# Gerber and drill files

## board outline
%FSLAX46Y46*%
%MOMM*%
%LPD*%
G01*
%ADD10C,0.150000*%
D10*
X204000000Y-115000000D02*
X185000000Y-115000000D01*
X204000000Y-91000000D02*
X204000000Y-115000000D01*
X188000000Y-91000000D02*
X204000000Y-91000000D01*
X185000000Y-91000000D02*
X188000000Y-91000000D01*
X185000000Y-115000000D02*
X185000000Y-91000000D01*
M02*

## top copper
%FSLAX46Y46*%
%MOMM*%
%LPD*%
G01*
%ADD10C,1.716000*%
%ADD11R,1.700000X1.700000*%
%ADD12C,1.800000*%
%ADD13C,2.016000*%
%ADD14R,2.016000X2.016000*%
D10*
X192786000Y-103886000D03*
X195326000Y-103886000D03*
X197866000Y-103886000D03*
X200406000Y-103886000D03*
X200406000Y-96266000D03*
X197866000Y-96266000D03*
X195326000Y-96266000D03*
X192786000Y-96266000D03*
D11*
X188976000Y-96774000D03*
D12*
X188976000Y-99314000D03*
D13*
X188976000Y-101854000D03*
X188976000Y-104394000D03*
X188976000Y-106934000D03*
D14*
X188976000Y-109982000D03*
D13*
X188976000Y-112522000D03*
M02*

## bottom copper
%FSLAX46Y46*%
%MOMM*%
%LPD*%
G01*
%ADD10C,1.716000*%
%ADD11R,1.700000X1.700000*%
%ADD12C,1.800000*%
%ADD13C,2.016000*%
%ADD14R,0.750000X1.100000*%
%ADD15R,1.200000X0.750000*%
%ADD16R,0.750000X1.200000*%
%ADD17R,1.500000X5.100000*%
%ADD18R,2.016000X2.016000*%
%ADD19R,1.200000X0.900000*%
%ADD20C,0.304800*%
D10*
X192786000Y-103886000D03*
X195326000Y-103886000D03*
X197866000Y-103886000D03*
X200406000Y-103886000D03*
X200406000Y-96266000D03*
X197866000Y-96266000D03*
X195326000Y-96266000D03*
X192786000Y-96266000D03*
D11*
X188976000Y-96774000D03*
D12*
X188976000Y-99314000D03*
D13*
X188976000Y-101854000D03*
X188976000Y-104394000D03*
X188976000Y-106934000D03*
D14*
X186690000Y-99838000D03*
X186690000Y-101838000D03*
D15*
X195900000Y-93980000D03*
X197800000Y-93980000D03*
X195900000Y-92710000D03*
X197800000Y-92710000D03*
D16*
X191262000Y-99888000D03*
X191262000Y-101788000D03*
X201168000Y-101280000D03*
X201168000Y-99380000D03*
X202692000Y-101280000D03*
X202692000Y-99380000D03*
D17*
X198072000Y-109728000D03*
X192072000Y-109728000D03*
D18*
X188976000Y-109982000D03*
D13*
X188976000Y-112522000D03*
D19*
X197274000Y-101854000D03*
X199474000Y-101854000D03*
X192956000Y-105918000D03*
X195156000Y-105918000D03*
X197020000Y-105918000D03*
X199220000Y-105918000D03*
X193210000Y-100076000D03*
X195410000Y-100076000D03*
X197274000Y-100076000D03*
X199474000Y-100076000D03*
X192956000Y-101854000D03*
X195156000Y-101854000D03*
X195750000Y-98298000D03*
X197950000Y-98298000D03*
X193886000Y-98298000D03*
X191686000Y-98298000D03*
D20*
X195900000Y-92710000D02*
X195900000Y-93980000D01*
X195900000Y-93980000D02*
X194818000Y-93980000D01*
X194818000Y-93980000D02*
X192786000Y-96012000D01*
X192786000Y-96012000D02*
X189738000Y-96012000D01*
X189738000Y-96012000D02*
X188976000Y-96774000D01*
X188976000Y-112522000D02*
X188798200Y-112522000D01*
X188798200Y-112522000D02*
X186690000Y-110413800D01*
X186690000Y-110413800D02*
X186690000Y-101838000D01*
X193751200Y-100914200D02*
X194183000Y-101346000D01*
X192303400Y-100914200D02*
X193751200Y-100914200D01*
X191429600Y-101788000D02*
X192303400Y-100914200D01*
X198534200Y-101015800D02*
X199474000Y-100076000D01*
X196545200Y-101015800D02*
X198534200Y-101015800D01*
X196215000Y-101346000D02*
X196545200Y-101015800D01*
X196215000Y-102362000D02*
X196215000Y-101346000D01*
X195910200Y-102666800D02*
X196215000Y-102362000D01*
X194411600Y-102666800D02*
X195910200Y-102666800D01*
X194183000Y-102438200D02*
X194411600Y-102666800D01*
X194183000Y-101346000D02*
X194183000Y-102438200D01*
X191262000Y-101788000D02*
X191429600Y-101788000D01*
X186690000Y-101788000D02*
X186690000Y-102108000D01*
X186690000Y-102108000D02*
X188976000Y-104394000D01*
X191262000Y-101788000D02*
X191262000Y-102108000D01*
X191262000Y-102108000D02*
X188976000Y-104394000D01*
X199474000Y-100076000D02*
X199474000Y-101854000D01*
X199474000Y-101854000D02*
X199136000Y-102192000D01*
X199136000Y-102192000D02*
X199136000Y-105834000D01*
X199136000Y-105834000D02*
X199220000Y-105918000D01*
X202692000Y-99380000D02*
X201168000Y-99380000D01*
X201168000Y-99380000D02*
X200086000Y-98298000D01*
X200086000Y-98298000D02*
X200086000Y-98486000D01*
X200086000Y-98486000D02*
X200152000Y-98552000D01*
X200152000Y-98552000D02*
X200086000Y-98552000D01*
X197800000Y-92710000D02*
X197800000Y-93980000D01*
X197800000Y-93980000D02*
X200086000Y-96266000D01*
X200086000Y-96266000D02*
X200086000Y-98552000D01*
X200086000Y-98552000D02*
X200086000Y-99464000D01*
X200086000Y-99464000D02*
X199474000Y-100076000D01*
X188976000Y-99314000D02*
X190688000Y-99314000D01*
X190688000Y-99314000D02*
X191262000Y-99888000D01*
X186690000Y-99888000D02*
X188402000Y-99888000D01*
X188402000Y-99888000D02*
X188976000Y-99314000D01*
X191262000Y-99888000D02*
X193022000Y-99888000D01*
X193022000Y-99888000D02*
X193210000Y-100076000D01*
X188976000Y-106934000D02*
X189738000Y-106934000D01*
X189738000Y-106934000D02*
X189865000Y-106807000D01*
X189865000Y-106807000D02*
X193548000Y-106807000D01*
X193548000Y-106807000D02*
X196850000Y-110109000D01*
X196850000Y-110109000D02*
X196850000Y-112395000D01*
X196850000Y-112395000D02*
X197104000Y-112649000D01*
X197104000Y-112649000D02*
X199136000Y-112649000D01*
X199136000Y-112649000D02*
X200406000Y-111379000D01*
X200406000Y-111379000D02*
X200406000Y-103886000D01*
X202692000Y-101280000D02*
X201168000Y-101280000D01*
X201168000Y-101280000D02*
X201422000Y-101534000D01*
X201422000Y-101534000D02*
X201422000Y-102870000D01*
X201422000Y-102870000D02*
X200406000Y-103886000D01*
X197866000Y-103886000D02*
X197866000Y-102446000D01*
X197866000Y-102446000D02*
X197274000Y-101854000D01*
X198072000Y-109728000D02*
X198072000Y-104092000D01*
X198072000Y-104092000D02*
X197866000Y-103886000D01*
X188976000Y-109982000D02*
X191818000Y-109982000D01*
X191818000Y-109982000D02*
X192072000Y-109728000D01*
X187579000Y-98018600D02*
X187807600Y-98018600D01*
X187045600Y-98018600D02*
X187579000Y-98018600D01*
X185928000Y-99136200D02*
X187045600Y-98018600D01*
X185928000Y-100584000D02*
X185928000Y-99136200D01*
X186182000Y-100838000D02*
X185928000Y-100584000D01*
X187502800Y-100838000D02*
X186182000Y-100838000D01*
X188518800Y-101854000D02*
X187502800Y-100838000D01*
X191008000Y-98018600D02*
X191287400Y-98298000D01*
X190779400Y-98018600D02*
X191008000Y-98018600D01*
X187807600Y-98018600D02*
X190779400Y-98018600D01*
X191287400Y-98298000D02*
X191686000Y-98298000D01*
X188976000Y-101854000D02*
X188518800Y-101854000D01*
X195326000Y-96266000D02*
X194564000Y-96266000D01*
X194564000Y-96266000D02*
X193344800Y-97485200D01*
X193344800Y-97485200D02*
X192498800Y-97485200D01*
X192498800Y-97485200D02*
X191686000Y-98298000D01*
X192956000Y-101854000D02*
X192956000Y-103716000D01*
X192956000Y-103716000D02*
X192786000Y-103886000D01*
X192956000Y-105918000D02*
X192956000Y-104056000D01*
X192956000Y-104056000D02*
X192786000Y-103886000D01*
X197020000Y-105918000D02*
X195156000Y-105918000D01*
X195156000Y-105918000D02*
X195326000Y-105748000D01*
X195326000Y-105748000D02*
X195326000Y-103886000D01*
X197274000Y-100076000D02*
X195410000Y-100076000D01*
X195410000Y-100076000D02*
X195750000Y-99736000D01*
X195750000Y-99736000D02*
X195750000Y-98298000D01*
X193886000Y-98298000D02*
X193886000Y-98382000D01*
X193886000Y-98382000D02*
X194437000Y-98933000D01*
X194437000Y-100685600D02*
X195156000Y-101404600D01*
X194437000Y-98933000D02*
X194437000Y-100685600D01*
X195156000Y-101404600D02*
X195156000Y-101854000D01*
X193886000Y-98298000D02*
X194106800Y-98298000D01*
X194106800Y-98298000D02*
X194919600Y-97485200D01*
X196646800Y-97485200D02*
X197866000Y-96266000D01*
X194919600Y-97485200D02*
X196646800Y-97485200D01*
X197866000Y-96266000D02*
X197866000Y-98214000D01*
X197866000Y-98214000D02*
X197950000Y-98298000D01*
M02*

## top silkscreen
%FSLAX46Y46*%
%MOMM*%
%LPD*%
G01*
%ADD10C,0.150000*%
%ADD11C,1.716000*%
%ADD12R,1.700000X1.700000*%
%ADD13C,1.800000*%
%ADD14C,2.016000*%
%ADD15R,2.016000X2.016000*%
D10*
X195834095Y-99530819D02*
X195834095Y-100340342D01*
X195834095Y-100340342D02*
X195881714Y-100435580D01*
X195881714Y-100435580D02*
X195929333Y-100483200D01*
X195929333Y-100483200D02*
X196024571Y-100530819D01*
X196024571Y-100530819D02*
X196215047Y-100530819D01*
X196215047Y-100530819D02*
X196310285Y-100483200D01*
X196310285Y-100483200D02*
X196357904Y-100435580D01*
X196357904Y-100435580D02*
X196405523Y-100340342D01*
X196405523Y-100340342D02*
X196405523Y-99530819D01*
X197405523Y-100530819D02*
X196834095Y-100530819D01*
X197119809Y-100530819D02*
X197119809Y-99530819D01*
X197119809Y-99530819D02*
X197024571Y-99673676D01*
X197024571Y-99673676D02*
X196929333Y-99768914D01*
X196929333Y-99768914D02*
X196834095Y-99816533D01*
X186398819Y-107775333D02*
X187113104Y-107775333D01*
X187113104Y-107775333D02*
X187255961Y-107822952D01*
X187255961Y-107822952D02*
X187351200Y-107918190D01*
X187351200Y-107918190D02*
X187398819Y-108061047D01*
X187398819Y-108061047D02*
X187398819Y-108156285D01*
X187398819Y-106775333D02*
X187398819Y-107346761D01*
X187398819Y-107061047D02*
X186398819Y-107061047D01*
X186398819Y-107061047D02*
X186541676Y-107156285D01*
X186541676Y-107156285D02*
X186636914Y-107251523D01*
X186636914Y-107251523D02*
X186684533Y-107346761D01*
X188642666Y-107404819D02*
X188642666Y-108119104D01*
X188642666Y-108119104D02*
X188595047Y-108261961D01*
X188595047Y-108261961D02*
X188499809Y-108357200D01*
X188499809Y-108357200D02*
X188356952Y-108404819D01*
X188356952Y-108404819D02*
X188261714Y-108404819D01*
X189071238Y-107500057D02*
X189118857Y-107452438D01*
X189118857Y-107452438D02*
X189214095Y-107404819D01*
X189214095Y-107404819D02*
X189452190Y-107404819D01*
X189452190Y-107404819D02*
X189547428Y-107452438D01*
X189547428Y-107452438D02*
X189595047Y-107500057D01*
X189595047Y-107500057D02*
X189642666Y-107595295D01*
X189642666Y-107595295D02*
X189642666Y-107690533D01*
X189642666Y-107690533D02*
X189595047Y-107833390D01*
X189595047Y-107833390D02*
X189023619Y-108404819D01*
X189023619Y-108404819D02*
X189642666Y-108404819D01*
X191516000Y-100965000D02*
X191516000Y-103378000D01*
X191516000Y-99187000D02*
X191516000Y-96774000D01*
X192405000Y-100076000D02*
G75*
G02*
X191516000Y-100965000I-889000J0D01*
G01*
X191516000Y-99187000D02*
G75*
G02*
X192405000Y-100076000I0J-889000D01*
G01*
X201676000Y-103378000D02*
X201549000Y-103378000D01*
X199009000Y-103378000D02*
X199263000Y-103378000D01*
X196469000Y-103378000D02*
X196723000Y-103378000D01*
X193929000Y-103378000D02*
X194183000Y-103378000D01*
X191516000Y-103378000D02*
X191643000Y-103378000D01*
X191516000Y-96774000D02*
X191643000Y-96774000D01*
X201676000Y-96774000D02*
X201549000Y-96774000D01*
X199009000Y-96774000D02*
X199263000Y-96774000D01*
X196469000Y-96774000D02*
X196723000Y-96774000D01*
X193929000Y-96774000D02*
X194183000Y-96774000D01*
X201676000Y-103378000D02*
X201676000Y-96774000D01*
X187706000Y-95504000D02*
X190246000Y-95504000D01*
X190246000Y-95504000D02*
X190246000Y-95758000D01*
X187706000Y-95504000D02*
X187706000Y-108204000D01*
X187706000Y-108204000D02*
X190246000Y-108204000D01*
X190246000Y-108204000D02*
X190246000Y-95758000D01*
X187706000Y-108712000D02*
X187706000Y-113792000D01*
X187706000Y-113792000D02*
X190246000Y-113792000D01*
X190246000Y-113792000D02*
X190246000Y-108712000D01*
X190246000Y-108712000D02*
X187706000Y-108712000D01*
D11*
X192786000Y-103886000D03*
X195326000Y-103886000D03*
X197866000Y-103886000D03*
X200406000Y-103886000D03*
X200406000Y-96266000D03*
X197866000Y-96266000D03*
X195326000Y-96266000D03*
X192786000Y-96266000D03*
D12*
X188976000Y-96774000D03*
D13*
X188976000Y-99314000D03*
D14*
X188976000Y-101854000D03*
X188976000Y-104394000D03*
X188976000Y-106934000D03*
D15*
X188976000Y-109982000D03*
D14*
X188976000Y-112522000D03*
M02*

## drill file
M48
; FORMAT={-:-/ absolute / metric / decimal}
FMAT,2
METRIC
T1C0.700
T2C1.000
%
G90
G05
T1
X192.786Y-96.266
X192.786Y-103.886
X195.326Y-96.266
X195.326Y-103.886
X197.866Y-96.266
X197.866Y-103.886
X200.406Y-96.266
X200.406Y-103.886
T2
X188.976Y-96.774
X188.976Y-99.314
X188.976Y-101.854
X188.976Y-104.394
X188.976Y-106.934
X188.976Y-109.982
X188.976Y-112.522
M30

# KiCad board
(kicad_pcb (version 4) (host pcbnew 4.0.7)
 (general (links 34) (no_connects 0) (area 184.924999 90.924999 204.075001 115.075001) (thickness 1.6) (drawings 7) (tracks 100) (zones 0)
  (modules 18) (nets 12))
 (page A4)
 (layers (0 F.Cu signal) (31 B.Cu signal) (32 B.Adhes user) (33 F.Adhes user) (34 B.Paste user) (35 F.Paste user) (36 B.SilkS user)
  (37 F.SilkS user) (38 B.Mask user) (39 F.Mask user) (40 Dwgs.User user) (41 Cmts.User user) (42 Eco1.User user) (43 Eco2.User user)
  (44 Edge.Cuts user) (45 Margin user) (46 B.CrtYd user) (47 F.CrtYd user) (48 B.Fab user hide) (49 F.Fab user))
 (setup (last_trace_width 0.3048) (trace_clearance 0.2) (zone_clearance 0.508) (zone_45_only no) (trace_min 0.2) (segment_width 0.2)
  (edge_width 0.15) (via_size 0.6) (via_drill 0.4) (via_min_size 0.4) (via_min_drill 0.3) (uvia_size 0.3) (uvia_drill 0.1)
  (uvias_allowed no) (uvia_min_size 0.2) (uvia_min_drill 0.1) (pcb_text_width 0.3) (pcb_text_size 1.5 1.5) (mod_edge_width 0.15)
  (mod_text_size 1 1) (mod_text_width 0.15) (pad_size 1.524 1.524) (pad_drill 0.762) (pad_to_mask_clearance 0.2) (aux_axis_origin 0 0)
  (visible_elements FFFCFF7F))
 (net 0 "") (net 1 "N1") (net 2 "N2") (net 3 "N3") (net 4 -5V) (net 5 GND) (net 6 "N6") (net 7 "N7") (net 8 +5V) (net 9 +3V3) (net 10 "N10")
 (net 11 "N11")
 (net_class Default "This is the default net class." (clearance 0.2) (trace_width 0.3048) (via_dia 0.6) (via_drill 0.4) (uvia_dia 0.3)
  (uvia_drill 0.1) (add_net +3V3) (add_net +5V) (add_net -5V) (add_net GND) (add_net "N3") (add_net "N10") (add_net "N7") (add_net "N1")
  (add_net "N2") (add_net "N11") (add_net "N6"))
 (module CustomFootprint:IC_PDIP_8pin (layer F.Cu) (at 196.596 100.076)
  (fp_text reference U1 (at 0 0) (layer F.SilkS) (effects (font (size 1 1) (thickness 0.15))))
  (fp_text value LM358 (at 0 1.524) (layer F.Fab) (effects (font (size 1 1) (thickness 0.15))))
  (fp_line (start -5.08 0.889) (end -5.08 3.302) (layer F.SilkS) (width 0.15))
  (fp_line (start -5.08 -0.889) (end -5.08 -3.302) (layer F.SilkS) (width 0.15))
  (fp_arc (start -5.08 0) (end -4.191 0) (angle 90) (layer F.SilkS) (width 0.15))
  (fp_arc (start -5.08 0) (end -5.08 -0.889) (angle 90) (layer F.SilkS) (width 0.15))
  (fp_line (start 5.08 3.302) (end 4.953 3.302) (layer F.SilkS) (width 0.15))
  (fp_line (start 2.413 3.302) (end 2.667 3.302) (layer F.SilkS) (width 0.15))
  (fp_line (start -0.127 3.302) (end 0.127 3.302) (layer F.SilkS) (width 0.15))
  (fp_line (start -2.667 3.302) (end -2.413 3.302) (layer F.SilkS) (width 0.15))
  (fp_line (start -5.08 3.302) (end -4.953 3.302) (layer F.SilkS) (width 0.15))
  (fp_line (start -5.08 -3.302) (end -4.953 -3.302) (layer F.SilkS) (width 0.15))
  (fp_line (start 5.08 -3.302) (end 4.953 -3.302) (layer F.SilkS) (width 0.15))
  (fp_line (start 2.413 -3.302) (end 2.667 -3.302) (layer F.SilkS) (width 0.15))
  (fp_line (start -0.127 -3.302) (end 0.127 -3.302) (layer F.SilkS) (width 0.15))
  (fp_line (start -2.667 -3.302) (end -2.413 -3.302) (layer F.SilkS) (width 0.15))
  (fp_line (start 5.08 3.302) (end 5.08 -3.302) (layer F.SilkS) (width 0.15))
  (pad 1 thru_hole circle (at -3.81 3.81) (size 1.716 1.716) (drill 0.7) (layers *.Cu *.Mask F.SilkS) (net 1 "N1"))
  (pad 2 thru_hole circle (at -1.27 3.81) (size 1.716 1.716) (drill 0.7) (layers *.Cu *.Mask F.SilkS) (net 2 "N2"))
  (pad 3 thru_hole circle (at 1.27 3.81) (size 1.716 1.716) (drill 0.7) (layers *.Cu *.Mask F.SilkS) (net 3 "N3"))
  (pad 4 thru_hole circle (at 3.81 3.81) (size 1.716 1.716) (drill 0.7) (layers *.Cu *.Mask F.SilkS) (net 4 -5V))
  (pad 5 thru_hole circle (at 3.81 -3.81) (size 1.716 1.716) (drill 0.7) (layers *.Cu *.Mask F.SilkS) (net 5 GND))
  (pad 6 thru_hole circle (at 1.27 -3.81) (size 1.716 1.716) (drill 0.7) (layers *.Cu *.Mask F.SilkS) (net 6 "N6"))
  (pad 7 thru_hole circle (at -1.27 -3.81) (size 1.716 1.716) (drill 0.7) (layers *.Cu *.Mask F.SilkS) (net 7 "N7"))
  (pad 8 thru_hole circle (at -3.81 -3.81) (size 1.716 1.716) (drill 0.7) (layers *.Cu *.Mask F.SilkS) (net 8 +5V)))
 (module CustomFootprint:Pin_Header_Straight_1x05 (layer F.Cu) (at 188.976 96.774)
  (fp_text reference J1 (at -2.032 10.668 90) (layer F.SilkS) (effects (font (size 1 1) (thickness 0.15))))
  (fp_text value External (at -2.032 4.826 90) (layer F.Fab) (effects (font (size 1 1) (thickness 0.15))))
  (fp_line (start -1.27 -1.27) (end 1.27 -1.27) (layer F.SilkS) (width 0.15))
  (fp_line (start 1.27 -1.27) (end 1.27 -1.016) (layer F.SilkS) (width 0.15))
  (fp_line (start -1.27 -1.27) (end -1.27 11.43) (layer F.SilkS) (width 0.15))
  (fp_line (start -1.27 11.43) (end 1.27 11.43) (layer F.SilkS) (width 0.15))
  (fp_line (start 1.27 11.43) (end 1.27 -1.016) (layer F.SilkS) (width 0.15))
  (pad 1 thru_hole rect (at 0 0) (size 1.7 1.7) (drill 1) (layers *.Cu *.Mask F.SilkS) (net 8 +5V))
  (pad 2 thru_hole circle (at 0 2.54) (size 1.8 1.8) (drill 1) (layers *.Cu *.Mask F.SilkS) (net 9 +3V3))
  (pad 3 thru_hole circle (at 0 5.08) (size 2.016 2.016) (drill 1) (layers *.Cu *.Mask F.SilkS) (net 7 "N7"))
  (pad 4 thru_hole circle (at 0 7.62) (size 2.016 2.016) (drill 1) (layers *.Cu *.Mask F.SilkS) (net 5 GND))
  (pad 5 thru_hole circle (at 0 10.16) (size 2.016 2.016) (drill 1) (layers *.Cu *.Mask F.SilkS) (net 4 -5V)))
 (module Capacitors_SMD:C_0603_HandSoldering (layer B.Cu) (at 186.69 100.838 270)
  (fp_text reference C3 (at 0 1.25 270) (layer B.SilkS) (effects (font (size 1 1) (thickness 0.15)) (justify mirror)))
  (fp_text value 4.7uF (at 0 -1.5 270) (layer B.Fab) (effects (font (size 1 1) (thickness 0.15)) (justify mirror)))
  (pad 1 smd rect (at -1 0 270) (size 1.1 0.75) (layers B.Cu B.Paste B.Mask) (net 9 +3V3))
  (pad 2 smd rect (at 1 0 270) (size 1.1 0.75) (layers B.Cu B.Paste B.Mask) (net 5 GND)))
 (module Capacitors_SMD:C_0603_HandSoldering (layer B.Cu) (at 196.85 93.98)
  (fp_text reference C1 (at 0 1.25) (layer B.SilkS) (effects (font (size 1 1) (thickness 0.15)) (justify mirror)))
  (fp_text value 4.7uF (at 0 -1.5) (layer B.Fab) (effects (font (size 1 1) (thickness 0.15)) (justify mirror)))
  (pad 1 smd rect (at -0.95 0) (size 1.2 0.75) (layers B.Cu B.Paste B.Mask) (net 8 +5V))
  (pad 2 smd rect (at 0.95 0) (size 1.2 0.75) (layers B.Cu B.Paste B.Mask) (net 5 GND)))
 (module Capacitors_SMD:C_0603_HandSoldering (layer B.Cu) (at 196.85 92.71)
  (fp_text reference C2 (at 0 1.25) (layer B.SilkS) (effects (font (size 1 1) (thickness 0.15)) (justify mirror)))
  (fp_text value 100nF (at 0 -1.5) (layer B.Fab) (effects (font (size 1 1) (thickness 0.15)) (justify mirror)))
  (pad 1 smd rect (at -0.95 0) (size 1.2 0.75) (layers B.Cu B.Paste B.Mask) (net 8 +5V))
  (pad 2 smd rect (at 0.95 0) (size 1.2 0.75) (layers B.Cu B.Paste B.Mask) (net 5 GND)))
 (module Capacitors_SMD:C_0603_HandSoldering (layer B.Cu) (at 191.262 100.838 270)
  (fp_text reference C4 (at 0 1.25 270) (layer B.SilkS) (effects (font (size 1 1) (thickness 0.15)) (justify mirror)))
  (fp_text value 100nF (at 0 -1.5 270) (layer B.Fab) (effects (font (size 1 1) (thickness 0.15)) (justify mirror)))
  (pad 1 smd rect (at -0.95 0 270) (size 1.2 0.75) (layers B.Cu B.Paste B.Mask) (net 9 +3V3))
  (pad 2 smd rect (at 0.95 0 270) (size 1.2 0.75) (layers B.Cu B.Paste B.Mask) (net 5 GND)))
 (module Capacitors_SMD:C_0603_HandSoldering (layer B.Cu) (at 201.168 100.33 90)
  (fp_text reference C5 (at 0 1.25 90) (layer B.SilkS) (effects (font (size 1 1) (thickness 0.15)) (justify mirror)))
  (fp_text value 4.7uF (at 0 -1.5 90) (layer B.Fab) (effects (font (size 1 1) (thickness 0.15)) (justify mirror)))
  (pad 1 smd rect (at -0.95 0 90) (size 1.2 0.75) (layers B.Cu B.Paste B.Mask) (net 4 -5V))
  (pad 2 smd rect (at 0.95 0 90) (size 1.2 0.75) (layers B.Cu B.Paste B.Mask) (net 5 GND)))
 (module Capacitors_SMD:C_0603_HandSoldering (layer B.Cu) (at 202.692 100.33 90)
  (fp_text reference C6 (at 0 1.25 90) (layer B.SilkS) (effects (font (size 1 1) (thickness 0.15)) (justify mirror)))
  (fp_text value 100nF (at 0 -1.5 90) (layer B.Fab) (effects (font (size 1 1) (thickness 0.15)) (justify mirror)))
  (pad 1 smd rect (at -0.95 0 90) (size 1.2 0.75) (layers B.Cu B.Paste B.Mask) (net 4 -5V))
  (pad 2 smd rect (at 0.95 0 90) (size 1.2 0.75) (layers B.Cu B.Paste B.Mask) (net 5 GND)))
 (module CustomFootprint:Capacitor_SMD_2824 (layer B.Cu) (at 195.072 109.728 180)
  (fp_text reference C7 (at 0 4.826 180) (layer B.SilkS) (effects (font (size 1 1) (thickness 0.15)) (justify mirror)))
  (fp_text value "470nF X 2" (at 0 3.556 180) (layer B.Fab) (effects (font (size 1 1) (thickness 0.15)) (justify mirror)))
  (pad 1 smd rect (at -3 0 180) (size 1.5 5.1) (layers B.Cu B.Paste B.Mask) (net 3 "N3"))
  (pad 2 smd rect (at 3 0 180) (size 1.5 5.1) (layers B.Cu B.Paste B.Mask) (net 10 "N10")))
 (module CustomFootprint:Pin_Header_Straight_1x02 (layer F.Cu) (at 188.976 109.982)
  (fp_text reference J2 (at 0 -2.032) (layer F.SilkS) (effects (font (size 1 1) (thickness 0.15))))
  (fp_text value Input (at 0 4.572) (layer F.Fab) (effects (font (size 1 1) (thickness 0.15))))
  (fp_line (start -1.27 -1.27) (end -1.27 3.81) (layer F.SilkS) (width 0.15))
  (fp_line (start -1.27 3.81) (end 1.27 3.81) (layer F.SilkS) (width 0.15))
  (fp_line (start 1.27 3.81) (end 1.27 -1.27) (layer F.SilkS) (width 0.15))
  (fp_line (start 1.27 -1.27) (end -1.27 -1.27) (layer F.SilkS) (width 0.15))
  (pad 1 thru_hole rect (at 0 0) (size 2.016 2.016) (drill 1) (layers *.Cu *.Mask F.SilkS) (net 10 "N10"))
  (pad 2 thru_hole circle (at 0 2.54) (size 2.016 2.016) (drill 1) (layers *.Cu *.Mask F.SilkS) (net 5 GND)))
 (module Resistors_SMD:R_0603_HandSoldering (layer B.Cu) (at 198.374 101.854)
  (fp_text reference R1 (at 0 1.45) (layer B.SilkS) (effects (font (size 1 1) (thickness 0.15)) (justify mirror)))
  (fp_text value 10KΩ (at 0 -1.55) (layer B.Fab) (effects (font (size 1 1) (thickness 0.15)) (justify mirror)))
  (pad 1 smd rect (at -1.1 0) (size 1.2 0.9) (layers B.Cu B.Paste B.Mask) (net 3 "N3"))
  (pad 2 smd rect (at 1.1 0) (size 1.2 0.9) (layers B.Cu B.Paste B.Mask) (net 5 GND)))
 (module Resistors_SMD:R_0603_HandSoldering (layer B.Cu) (at 194.056 105.918)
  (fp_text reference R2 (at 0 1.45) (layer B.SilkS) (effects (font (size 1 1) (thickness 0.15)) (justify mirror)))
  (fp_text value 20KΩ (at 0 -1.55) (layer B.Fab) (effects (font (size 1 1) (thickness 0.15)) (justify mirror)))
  (pad 1 smd rect (at -1.1 0) (size 1.2 0.9) (layers B.Cu B.Paste B.Mask) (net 1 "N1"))
  (pad 2 smd rect (at 1.1 0) (size 1.2 0.9) (layers B.Cu B.Paste B.Mask) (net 2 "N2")))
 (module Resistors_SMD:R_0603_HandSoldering (layer B.Cu) (at 198.12 105.918)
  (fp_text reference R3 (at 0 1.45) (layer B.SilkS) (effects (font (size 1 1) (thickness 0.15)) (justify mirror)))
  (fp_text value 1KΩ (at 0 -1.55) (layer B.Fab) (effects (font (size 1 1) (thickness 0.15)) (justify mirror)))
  (pad 1 smd rect (at -1.1 0) (size 1.2 0.9) (layers B.Cu B.Paste B.Mask) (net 2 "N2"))
  (pad 2 smd rect (at 1.1 0) (size 1.2 0.9) (layers B.Cu B.Paste B.Mask) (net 5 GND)))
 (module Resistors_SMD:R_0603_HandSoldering (layer B.Cu) (at 194.31 100.076)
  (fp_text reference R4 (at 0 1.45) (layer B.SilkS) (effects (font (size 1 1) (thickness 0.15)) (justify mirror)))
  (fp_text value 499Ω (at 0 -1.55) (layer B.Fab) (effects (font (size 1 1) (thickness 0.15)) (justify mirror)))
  (pad 1 smd rect (at -1.1 0) (size 1.2 0.9) (layers B.Cu B.Paste B.Mask) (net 9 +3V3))
  (pad 2 smd rect (at 1.1 0) (size 1.2 0.9) (layers B.Cu B.Paste B.Mask) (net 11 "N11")))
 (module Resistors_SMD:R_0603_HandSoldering (layer B.Cu) (at 198.374 100.076)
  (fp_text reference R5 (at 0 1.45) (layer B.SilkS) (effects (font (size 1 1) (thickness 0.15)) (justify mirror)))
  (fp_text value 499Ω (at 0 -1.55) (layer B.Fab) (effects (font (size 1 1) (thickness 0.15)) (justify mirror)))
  (pad 1 smd rect (at -1.1 0) (size 1.2 0.9) (layers B.Cu B.Paste B.Mask) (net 11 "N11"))
  (pad 2 smd rect (at 1.1 0) (size 1.2 0.9) (layers B.Cu B.Paste B.Mask) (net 5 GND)))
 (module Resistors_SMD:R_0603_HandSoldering (layer B.Cu) (at 194.056 101.854)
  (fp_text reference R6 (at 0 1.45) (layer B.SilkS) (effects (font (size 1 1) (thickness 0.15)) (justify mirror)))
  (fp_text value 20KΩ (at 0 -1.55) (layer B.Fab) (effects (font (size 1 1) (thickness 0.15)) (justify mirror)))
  (pad 1 smd rect (at -1.1 0) (size 1.2 0.9) (layers B.Cu B.Paste B.Mask) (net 1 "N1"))
  (pad 2 smd rect (at 1.1 0) (size 1.2 0.9) (layers B.Cu B.Paste B.Mask) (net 6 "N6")))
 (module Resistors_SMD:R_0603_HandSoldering (layer B.Cu) (at 196.85 98.298)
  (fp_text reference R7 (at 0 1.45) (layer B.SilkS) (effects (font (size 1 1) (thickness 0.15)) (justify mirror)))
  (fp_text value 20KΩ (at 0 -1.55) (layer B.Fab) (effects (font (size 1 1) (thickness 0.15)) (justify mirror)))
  (pad 1 smd rect (at -1.1 0) (size 1.2 0.9) (layers B.Cu B.Paste B.Mask) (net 11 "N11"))
  (pad 2 smd rect (at 1.1 0) (size 1.2 0.9) (layers B.Cu B.Paste B.Mask) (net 6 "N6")))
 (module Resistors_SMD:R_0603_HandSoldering (layer B.Cu) (at 192.786 98.298 180)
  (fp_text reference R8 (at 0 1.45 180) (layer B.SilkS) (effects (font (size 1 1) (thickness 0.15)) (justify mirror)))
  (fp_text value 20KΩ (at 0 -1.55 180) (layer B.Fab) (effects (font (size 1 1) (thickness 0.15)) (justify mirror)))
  (pad 1 smd rect (at -1.1 0 180) (size 1.2 0.9) (layers B.Cu B.Paste B.Mask) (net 6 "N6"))
  (pad 2 smd rect (at 1.1 0 180) (size 1.2 0.9) (layers B.Cu B.Paste B.Mask) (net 7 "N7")))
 (gr_line (start 204 115) (end 185 115) (angle 90) (layer Edge.Cuts) (width 0.15))
 (gr_line (start 204 91) (end 204 115) (angle 90) (layer Edge.Cuts) (width 0.15))
 (gr_line (start 188 91) (end 204 91) (angle 90) (layer Edge.Cuts) (width 0.15))
 (gr_line (start 185 91) (end 188 91) (angle 90) (layer Edge.Cuts) (width 0.15))
 (gr_line (start 185 115) (end 185 91) (angle 90) (layer Edge.Cuts) (width 0.15))
 (segment (start 195.9 92.71) (end 195.9 93.98) (width 0.3048) (layer B.Cu) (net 8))
 (segment (start 195.9 93.98) (end 194.818 93.98) (width 0.3048) (layer B.Cu) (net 8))
 (segment (start 194.818 93.98) (end 192.786 96.012) (width 0.3048) (layer B.Cu) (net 8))
 (segment (start 192.786 96.012) (end 189.738 96.012) (width 0.3048) (layer B.Cu) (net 8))
 (segment (start 189.738 96.012) (end 188.976 96.774) (width 0.3048) (layer B.Cu) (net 8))
 (segment (start 188.976 112.522) (end 188.7982 112.522) (width 0.3048) (layer B.Cu) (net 5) (status C00000))
 (segment (start 188.7982 112.522) (end 186.69 110.4138) (width 0.3048) (layer B.Cu) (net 5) (status 400000))
 (segment (start 186.69 110.4138) (end 186.69 101.838) (width 0.3048) (layer B.Cu) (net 5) (status 800000))
 (segment (start 193.7512 100.9142) (end 194.183 101.346) (width 0.3048) (layer B.Cu) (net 5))
 (segment (start 192.3034 100.9142) (end 193.7512 100.9142) (width 0.3048) (layer B.Cu) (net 5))
 (segment (start 191.4296 101.788) (end 192.3034 100.9142) (width 0.3048) (layer B.Cu) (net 5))
 (segment (start 198.5342 101.0158) (end 199.474 100.076) (width 0.3048) (layer B.Cu) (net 5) (status 800000))
 (segment (start 196.5452 101.0158) (end 198.5342 101.0158) (width 0.3048) (layer B.Cu) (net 5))
 (segment (start 196.215 101.346) (end 196.5452 101.0158) (width 0.3048) (layer B.Cu) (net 5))
 (segment (start 196.215 102.362) (end 196.215 101.346) (width 0.3048) (layer B.Cu) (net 5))
 (segment (start 195.9102 102.6668) (end 196.215 102.362) (width 0.3048) (layer B.Cu) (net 5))
 (segment (start 194.4116 102.6668) (end 195.9102 102.6668) (width 0.3048) (layer B.Cu) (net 5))
 (segment (start 194.183 102.4382) (end 194.4116 102.6668) (width 0.3048) (layer B.Cu) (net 5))
 (segment (start 194.183 101.346) (end 194.183 102.4382) (width 0.3048) (layer B.Cu) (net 5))
 (segment (start 191.262 101.788) (end 191.4296 101.788) (width 0.3048) (layer B.Cu) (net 5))
 (segment (start 186.69 101.788) (end 186.69 102.108) (width 0.3048) (layer B.Cu) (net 5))
 (segment (start 186.69 102.108) (end 188.976 104.394) (width 0.3048) (layer B.Cu) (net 5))
 (segment (start 191.262 101.788) (end 191.262 102.108) (width 0.3048) (layer B.Cu) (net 5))
 (segment (start 191.262 102.108) (end 188.976 104.394) (width 0.3048) (layer B.Cu) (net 5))
 (segment (start 199.474 100.076) (end 199.474 101.854) (width 0.3048) (layer B.Cu) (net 5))
 (segment (start 199.474 101.854) (end 199.136 102.192) (width 0.3048) (layer B.Cu) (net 5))
 (segment (start 199.136 102.192) (end 199.136 105.834) (width 0.3048) (layer B.Cu) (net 5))
 (segment (start 199.136 105.834) (end 199.22 105.918) (width 0.3048) (layer B.Cu) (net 5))
 (segment (start 202.692 99.38) (end 201.168 99.38) (width 0.3048) (layer B.Cu) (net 5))
 (segment (start 201.168 99.38) (end 200.086 98.298) (width 0.3048) (layer B.Cu) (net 5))
 (segment (start 200.086 98.298) (end 200.086 98.486) (width 0.3048) (layer B.Cu) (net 5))
 (segment (start 200.086 98.486) (end 200.152 98.552) (width 0.3048) (layer B.Cu) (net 5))
 (segment (start 200.152 98.552) (end 200.086 98.552) (width 0.3048) (layer B.Cu) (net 5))
 (segment (start 197.8 92.71) (end 197.8 93.98) (width 0.3048) (layer B.Cu) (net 5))
 (segment (start 197.8 93.98) (end 200.086 96.266) (width 0.3048) (layer B.Cu) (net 5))
 (segment (start 200.086 96.266) (end 200.086 98.552) (width 0.3048) (layer B.Cu) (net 5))
 (segment (start 200.086 98.552) (end 200.086 99.464) (width 0.3048) (layer B.Cu) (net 5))
 (segment (start 200.086 99.464) (end 199.474 100.076) (width 0.3048) (layer B.Cu) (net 5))
 (segment (start 188.976 99.314) (end 190.688 99.314) (width 0.3048) (layer B.Cu) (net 9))
 (segment (start 190.688 99.314) (end 191.262 99.888) (width 0.3048) (layer B.Cu) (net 9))
 (segment (start 186.69 99.888) (end 188.402 99.888) (width 0.3048) (layer B.Cu) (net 9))
 (segment (start 188.402 99.888) (end 188.976 99.314) (width 0.3048) (layer B.Cu) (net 9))
 (segment (start 191.262 99.888) (end 193.022 99.888) (width 0.3048) (layer B.Cu) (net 9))
 (segment (start 193.022 99.888) (end 193.21 100.076) (width 0.3048) (layer B.Cu) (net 9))
 (segment (start 188.976 106.934) (end 189.738 106.934) (width 0.3048) (layer B.Cu) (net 4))
 (segment (start 189.738 106.934) (end 189.865 106.807) (width 0.3048) (layer B.Cu) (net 4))
 (segment (start 189.865 106.807) (end 193.548 106.807) (width 0.3048) (layer B.Cu) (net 4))
 (segment (start 193.548 106.807) (end 196.85 110.109) (width 0.3048) (layer B.Cu) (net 4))
 (segment (start 196.85 110.109) (end 196.85 112.395) (width 0.3048) (layer B.Cu) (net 4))
 (segment (start 196.85 112.395) (end 197.104 112.649) (width 0.3048) (layer B.Cu) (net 4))
 (segment (start 197.104 112.649) (end 199.136 112.649) (width 0.3048) (layer B.Cu) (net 4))
 (segment (start 199.136 112.649) (end 200.406 111.379) (width 0.3048) (layer B.Cu) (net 4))
 (segment (start 200.406 111.379) (end 200.406 103.886) (width 0.3048) (layer B.Cu) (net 4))
 (segment (start 202.692 101.28) (end 201.168 101.28) (width 0.3048) (layer B.Cu) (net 4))
 (segment (start 201.168 101.28) (end 201.422 101.534) (width 0.3048) (layer B.Cu) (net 4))
 (segment (start 201.422 101.534) (end 201.422 102.87) (width 0.3048) (layer B.Cu) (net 4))
 (segment (start 201.422 102.87) (end 200.406 103.886) (width 0.3048) (layer B.Cu) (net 4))
 (segment (start 197.866 103.886) (end 197.866 102.446) (width 0.3048) (layer B.Cu) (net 3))
 (segment (start 197.866 102.446) (end 197.274 101.854) (width 0.3048) (layer B.Cu) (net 3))
 (segment (start 198.072 109.728) (end 198.072 104.092) (width 0.3048) (layer B.Cu) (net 3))
 (segment (start 198.072 104.092) (end 197.866 103.886) (width 0.3048) (layer B.Cu) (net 3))
 (segment (start 188.976 109.982) (end 191.818 109.982) (width 0.3048) (layer B.Cu) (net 10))
 (segment (start 191.818 109.982) (end 192.072 109.728) (width 0.3048) (layer B.Cu) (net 10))
 (segment (start 187.579 98.0186) (end 187.8076 98.0186) (width 0.3048) (layer B.Cu) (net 7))
 (segment (start 187.0456 98.0186) (end 187.579 98.0186) (width 0.3048) (layer B.Cu) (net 7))
 (segment (start 185.928 99.1362) (end 187.0456 98.0186) (width 0.3048) (layer B.Cu) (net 7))
 (segment (start 185.928 100.584) (end 185.928 99.1362) (width 0.3048) (layer B.Cu) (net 7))
 (segment (start 186.182 100.838) (end 185.928 100.584) (width 0.3048) (layer B.Cu) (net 7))
 (segment (start 187.5028 100.838) (end 186.182 100.838) (width 0.3048) (layer B.Cu) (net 7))
 (segment (start 188.5188 101.854) (end 187.5028 100.838) (width 0.3048) (layer B.Cu) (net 7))
 (segment (start 191.008 98.0186) (end 191.2874 98.298) (width 0.3048) (layer B.Cu) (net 7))
 (segment (start 190.7794 98.0186) (end 191.008 98.0186) (width 0.3048) (layer B.Cu) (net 7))
 (segment (start 187.8076 98.0186) (end 190.7794 98.0186) (width 0.3048) (layer B.Cu) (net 7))
 (segment (start 191.2874 98.298) (end 191.686 98.298) (width 0.3048) (layer B.Cu) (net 7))
 (segment (start 188.976 101.854) (end 188.5188 101.854) (width 0.3048) (layer B.Cu) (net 7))
 (segment (start 195.326 96.266) (end 194.564 96.266) (width 0.3048) (layer B.Cu) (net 7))
 (segment (start 194.564 96.266) (end 193.3448 97.4852) (width 0.3048) (layer B.Cu) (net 7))
 (segment (start 193.3448 97.4852) (end 192.4988 97.4852) (width 0.3048) (layer B.Cu) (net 7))
 (segment (start 192.4988 97.4852) (end 191.686 98.298) (width 0.3048) (layer B.Cu) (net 7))
 (segment (start 192.956 101.854) (end 192.956 103.716) (width 0.3048) (layer B.Cu) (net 1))
 (segment (start 192.956 103.716) (end 192.786 103.886) (width 0.3048) (layer B.Cu) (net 1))
 (segment (start 192.956 105.918) (end 192.956 104.056) (width 0.3048) (layer B.Cu) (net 1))
 (segment (start 192.956 104.056) (end 192.786 103.886) (width 0.3048) (layer B.Cu) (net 1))
 (segment (start 197.02 105.918) (end 195.156 105.918) (width 0.3048) (layer B.Cu) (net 2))
 (segment (start 195.156 105.918) (end 195.326 105.748) (width 0.3048) (layer B.Cu) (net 2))
 (segment (start 195.326 105.748) (end 195.326 103.886) (width 0.3048) (layer B.Cu) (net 2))
 (segment (start 197.274 100.076) (end 195.41 100.076) (width 0.3048) (layer B.Cu) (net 11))
 (segment (start 195.41 100.076) (end 195.75 99.736) (width 0.3048) (layer B.Cu) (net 11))
 (segment (start 195.75 99.736) (end 195.75 98.298) (width 0.3048) (layer B.Cu) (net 11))
 (segment (start 193.886 98.298) (end 193.886 98.382) (width 0.3048) (layer B.Cu) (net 6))
 (segment (start 193.886 98.382) (end 194.437 98.933) (width 0.3048) (layer B.Cu) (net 6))
 (segment (start 194.437 100.6856) (end 195.156 101.4046) (width 0.3048) (layer B.Cu) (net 6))
 (segment (start 194.437 98.933) (end 194.437 100.6856) (width 0.3048) (layer B.Cu) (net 6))
 (segment (start 195.156 101.4046) (end 195.156 101.854) (width 0.3048) (layer B.Cu) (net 6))
 (segment (start 193.886 98.298) (end 194.1068 98.298) (width 0.3048) (layer B.Cu) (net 6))
 (segment (start 194.1068 98.298) (end 194.9196 97.4852) (width 0.3048) (layer B.Cu) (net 6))
 (segment (start 196.6468 97.4852) (end 197.866 96.266) (width 0.3048) (layer B.Cu) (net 6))
 (segment (start 194.9196 97.4852) (end 196.6468 97.4852) (width 0.3048) (layer B.Cu) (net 6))
 (segment (start 197.866 96.266) (end 197.866 98.214) (width 0.3048) (layer B.Cu) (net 6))
 (segment (start 197.866 98.214) (end 197.95 98.298) (width 0.3048) (layer B.Cu) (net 6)))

